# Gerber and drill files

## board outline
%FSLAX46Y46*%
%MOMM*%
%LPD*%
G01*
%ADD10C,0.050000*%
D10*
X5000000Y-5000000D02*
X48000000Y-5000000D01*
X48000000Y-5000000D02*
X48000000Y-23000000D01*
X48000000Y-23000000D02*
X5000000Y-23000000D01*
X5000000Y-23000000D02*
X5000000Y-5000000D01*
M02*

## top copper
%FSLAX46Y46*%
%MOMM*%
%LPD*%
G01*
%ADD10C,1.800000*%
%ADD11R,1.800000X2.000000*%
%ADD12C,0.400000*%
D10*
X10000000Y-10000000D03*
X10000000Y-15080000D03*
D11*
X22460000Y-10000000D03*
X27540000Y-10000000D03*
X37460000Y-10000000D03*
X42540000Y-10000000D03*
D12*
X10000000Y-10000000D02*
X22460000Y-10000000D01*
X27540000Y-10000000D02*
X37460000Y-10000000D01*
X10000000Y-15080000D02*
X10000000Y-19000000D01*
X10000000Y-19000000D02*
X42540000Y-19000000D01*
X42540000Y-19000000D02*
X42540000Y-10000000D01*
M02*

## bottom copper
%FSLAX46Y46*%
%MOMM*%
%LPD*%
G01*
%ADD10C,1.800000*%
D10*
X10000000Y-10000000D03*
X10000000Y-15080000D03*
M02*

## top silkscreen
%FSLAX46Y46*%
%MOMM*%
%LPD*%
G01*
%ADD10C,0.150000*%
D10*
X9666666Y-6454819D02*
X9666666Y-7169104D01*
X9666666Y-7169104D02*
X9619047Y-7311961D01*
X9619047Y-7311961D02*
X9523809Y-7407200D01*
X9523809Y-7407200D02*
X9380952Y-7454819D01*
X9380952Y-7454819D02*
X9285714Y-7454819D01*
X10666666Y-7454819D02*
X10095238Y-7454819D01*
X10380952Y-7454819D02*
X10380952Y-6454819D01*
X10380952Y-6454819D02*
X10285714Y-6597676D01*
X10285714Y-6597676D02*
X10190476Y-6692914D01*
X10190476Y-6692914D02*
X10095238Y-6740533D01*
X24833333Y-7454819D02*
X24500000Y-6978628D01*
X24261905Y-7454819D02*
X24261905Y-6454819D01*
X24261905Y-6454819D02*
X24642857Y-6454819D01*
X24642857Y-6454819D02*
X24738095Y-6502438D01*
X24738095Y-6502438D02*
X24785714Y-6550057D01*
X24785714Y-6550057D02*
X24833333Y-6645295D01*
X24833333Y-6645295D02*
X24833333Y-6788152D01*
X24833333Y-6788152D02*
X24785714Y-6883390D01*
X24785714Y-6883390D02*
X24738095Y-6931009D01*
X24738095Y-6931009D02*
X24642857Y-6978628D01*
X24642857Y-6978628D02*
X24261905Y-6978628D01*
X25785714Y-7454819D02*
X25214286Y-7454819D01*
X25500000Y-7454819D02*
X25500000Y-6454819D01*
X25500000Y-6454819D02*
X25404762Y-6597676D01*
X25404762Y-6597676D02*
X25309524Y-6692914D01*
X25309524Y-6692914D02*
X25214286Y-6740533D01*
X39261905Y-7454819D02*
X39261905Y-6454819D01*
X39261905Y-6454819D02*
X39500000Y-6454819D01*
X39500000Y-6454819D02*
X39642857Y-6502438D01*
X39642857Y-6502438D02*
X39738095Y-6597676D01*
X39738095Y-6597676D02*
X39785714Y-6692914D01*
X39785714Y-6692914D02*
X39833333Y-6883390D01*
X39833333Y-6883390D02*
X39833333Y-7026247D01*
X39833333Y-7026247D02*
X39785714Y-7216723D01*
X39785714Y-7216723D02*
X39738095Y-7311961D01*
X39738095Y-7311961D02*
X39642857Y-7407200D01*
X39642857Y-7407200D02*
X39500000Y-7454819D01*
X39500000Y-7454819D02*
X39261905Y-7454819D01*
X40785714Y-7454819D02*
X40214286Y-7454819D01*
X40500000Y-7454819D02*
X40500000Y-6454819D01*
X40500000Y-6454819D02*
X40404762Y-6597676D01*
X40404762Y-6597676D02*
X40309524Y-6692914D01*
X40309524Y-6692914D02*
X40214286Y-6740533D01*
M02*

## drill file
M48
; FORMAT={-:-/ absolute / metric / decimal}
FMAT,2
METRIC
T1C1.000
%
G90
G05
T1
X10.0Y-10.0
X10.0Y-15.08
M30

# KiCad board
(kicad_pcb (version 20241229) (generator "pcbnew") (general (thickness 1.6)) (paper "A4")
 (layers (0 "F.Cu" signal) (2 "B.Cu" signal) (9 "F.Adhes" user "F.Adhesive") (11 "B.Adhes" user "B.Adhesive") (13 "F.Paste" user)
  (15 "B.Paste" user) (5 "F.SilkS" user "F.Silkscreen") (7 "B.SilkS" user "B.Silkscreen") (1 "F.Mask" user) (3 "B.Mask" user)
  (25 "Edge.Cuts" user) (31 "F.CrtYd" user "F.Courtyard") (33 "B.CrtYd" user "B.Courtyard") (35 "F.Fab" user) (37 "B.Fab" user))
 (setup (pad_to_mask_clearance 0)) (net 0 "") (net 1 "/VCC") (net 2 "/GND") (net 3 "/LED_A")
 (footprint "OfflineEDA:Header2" (layer "F.Cu") (at 10 10)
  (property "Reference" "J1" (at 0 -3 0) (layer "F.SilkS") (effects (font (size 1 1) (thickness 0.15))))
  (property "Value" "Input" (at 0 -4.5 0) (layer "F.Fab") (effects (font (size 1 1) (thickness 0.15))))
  (pad "1" thru_hole circle (at 0 0) (size 1.8 1.8) (drill 1) (layers "*.Cu" "*.Mask") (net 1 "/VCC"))
  (pad "2" thru_hole circle (at 0 5.08) (size 1.8 1.8) (drill 1) (layers "*.Cu" "*.Mask") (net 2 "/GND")))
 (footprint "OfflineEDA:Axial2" (layer "F.Cu") (at 25 10)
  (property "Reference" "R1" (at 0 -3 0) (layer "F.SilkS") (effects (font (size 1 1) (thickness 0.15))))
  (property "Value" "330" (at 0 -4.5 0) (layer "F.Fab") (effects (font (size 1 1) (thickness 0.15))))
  (pad "1" smd rect (at -2.54 0) (size 1.8 2) (layers "F.Cu" "F.Paste" "F.Mask") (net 1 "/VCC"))
  (pad "2" smd rect (at 2.54 0) (size 1.8 2) (layers "F.Cu" "F.Paste" "F.Mask") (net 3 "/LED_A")))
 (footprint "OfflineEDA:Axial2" (layer "F.Cu") (at 40 10)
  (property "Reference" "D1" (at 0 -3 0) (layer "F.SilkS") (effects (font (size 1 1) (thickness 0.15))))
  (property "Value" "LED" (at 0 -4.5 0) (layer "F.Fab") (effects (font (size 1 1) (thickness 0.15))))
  (pad "1" smd rect (at -2.54 0) (size 1.8 2) (layers "F.Cu" "F.Paste" "F.Mask") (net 3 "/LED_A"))
  (pad "2" smd rect (at 2.54 0) (size 1.8 2) (layers "F.Cu" "F.Paste" "F.Mask") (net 2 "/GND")))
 (segment (start 10 10) (end 22.46 10) (width 0.4) (layer "F.Cu") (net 1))
 (segment (start 27.54 10) (end 37.46 10) (width 0.4) (layer "F.Cu") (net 3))
 (segment (start 10 15.08) (end 10 19) (width 0.4) (layer "F.Cu") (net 2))
 (segment (start 10 19) (end 42.54 19) (width 0.4) (layer "F.Cu") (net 2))
 (segment (start 42.54 19) (end 42.54 10) (width 0.4) (layer "F.Cu") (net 2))
 (gr_line (start 5 5) (end 48 5) (stroke (width 0.05) (type default)) (layer "Edge.Cuts"))
 (gr_line (start 48 5) (end 48 23) (stroke (width 0.05) (type default)) (layer "Edge.Cuts"))
 (gr_line (start 48 23) (end 5 23) (stroke (width 0.05) (type default)) (layer "Edge.Cuts"))
 (gr_line (start 5 23) (end 5 5) (stroke (width 0.05) (type default)) (layer "Edge.Cuts")))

